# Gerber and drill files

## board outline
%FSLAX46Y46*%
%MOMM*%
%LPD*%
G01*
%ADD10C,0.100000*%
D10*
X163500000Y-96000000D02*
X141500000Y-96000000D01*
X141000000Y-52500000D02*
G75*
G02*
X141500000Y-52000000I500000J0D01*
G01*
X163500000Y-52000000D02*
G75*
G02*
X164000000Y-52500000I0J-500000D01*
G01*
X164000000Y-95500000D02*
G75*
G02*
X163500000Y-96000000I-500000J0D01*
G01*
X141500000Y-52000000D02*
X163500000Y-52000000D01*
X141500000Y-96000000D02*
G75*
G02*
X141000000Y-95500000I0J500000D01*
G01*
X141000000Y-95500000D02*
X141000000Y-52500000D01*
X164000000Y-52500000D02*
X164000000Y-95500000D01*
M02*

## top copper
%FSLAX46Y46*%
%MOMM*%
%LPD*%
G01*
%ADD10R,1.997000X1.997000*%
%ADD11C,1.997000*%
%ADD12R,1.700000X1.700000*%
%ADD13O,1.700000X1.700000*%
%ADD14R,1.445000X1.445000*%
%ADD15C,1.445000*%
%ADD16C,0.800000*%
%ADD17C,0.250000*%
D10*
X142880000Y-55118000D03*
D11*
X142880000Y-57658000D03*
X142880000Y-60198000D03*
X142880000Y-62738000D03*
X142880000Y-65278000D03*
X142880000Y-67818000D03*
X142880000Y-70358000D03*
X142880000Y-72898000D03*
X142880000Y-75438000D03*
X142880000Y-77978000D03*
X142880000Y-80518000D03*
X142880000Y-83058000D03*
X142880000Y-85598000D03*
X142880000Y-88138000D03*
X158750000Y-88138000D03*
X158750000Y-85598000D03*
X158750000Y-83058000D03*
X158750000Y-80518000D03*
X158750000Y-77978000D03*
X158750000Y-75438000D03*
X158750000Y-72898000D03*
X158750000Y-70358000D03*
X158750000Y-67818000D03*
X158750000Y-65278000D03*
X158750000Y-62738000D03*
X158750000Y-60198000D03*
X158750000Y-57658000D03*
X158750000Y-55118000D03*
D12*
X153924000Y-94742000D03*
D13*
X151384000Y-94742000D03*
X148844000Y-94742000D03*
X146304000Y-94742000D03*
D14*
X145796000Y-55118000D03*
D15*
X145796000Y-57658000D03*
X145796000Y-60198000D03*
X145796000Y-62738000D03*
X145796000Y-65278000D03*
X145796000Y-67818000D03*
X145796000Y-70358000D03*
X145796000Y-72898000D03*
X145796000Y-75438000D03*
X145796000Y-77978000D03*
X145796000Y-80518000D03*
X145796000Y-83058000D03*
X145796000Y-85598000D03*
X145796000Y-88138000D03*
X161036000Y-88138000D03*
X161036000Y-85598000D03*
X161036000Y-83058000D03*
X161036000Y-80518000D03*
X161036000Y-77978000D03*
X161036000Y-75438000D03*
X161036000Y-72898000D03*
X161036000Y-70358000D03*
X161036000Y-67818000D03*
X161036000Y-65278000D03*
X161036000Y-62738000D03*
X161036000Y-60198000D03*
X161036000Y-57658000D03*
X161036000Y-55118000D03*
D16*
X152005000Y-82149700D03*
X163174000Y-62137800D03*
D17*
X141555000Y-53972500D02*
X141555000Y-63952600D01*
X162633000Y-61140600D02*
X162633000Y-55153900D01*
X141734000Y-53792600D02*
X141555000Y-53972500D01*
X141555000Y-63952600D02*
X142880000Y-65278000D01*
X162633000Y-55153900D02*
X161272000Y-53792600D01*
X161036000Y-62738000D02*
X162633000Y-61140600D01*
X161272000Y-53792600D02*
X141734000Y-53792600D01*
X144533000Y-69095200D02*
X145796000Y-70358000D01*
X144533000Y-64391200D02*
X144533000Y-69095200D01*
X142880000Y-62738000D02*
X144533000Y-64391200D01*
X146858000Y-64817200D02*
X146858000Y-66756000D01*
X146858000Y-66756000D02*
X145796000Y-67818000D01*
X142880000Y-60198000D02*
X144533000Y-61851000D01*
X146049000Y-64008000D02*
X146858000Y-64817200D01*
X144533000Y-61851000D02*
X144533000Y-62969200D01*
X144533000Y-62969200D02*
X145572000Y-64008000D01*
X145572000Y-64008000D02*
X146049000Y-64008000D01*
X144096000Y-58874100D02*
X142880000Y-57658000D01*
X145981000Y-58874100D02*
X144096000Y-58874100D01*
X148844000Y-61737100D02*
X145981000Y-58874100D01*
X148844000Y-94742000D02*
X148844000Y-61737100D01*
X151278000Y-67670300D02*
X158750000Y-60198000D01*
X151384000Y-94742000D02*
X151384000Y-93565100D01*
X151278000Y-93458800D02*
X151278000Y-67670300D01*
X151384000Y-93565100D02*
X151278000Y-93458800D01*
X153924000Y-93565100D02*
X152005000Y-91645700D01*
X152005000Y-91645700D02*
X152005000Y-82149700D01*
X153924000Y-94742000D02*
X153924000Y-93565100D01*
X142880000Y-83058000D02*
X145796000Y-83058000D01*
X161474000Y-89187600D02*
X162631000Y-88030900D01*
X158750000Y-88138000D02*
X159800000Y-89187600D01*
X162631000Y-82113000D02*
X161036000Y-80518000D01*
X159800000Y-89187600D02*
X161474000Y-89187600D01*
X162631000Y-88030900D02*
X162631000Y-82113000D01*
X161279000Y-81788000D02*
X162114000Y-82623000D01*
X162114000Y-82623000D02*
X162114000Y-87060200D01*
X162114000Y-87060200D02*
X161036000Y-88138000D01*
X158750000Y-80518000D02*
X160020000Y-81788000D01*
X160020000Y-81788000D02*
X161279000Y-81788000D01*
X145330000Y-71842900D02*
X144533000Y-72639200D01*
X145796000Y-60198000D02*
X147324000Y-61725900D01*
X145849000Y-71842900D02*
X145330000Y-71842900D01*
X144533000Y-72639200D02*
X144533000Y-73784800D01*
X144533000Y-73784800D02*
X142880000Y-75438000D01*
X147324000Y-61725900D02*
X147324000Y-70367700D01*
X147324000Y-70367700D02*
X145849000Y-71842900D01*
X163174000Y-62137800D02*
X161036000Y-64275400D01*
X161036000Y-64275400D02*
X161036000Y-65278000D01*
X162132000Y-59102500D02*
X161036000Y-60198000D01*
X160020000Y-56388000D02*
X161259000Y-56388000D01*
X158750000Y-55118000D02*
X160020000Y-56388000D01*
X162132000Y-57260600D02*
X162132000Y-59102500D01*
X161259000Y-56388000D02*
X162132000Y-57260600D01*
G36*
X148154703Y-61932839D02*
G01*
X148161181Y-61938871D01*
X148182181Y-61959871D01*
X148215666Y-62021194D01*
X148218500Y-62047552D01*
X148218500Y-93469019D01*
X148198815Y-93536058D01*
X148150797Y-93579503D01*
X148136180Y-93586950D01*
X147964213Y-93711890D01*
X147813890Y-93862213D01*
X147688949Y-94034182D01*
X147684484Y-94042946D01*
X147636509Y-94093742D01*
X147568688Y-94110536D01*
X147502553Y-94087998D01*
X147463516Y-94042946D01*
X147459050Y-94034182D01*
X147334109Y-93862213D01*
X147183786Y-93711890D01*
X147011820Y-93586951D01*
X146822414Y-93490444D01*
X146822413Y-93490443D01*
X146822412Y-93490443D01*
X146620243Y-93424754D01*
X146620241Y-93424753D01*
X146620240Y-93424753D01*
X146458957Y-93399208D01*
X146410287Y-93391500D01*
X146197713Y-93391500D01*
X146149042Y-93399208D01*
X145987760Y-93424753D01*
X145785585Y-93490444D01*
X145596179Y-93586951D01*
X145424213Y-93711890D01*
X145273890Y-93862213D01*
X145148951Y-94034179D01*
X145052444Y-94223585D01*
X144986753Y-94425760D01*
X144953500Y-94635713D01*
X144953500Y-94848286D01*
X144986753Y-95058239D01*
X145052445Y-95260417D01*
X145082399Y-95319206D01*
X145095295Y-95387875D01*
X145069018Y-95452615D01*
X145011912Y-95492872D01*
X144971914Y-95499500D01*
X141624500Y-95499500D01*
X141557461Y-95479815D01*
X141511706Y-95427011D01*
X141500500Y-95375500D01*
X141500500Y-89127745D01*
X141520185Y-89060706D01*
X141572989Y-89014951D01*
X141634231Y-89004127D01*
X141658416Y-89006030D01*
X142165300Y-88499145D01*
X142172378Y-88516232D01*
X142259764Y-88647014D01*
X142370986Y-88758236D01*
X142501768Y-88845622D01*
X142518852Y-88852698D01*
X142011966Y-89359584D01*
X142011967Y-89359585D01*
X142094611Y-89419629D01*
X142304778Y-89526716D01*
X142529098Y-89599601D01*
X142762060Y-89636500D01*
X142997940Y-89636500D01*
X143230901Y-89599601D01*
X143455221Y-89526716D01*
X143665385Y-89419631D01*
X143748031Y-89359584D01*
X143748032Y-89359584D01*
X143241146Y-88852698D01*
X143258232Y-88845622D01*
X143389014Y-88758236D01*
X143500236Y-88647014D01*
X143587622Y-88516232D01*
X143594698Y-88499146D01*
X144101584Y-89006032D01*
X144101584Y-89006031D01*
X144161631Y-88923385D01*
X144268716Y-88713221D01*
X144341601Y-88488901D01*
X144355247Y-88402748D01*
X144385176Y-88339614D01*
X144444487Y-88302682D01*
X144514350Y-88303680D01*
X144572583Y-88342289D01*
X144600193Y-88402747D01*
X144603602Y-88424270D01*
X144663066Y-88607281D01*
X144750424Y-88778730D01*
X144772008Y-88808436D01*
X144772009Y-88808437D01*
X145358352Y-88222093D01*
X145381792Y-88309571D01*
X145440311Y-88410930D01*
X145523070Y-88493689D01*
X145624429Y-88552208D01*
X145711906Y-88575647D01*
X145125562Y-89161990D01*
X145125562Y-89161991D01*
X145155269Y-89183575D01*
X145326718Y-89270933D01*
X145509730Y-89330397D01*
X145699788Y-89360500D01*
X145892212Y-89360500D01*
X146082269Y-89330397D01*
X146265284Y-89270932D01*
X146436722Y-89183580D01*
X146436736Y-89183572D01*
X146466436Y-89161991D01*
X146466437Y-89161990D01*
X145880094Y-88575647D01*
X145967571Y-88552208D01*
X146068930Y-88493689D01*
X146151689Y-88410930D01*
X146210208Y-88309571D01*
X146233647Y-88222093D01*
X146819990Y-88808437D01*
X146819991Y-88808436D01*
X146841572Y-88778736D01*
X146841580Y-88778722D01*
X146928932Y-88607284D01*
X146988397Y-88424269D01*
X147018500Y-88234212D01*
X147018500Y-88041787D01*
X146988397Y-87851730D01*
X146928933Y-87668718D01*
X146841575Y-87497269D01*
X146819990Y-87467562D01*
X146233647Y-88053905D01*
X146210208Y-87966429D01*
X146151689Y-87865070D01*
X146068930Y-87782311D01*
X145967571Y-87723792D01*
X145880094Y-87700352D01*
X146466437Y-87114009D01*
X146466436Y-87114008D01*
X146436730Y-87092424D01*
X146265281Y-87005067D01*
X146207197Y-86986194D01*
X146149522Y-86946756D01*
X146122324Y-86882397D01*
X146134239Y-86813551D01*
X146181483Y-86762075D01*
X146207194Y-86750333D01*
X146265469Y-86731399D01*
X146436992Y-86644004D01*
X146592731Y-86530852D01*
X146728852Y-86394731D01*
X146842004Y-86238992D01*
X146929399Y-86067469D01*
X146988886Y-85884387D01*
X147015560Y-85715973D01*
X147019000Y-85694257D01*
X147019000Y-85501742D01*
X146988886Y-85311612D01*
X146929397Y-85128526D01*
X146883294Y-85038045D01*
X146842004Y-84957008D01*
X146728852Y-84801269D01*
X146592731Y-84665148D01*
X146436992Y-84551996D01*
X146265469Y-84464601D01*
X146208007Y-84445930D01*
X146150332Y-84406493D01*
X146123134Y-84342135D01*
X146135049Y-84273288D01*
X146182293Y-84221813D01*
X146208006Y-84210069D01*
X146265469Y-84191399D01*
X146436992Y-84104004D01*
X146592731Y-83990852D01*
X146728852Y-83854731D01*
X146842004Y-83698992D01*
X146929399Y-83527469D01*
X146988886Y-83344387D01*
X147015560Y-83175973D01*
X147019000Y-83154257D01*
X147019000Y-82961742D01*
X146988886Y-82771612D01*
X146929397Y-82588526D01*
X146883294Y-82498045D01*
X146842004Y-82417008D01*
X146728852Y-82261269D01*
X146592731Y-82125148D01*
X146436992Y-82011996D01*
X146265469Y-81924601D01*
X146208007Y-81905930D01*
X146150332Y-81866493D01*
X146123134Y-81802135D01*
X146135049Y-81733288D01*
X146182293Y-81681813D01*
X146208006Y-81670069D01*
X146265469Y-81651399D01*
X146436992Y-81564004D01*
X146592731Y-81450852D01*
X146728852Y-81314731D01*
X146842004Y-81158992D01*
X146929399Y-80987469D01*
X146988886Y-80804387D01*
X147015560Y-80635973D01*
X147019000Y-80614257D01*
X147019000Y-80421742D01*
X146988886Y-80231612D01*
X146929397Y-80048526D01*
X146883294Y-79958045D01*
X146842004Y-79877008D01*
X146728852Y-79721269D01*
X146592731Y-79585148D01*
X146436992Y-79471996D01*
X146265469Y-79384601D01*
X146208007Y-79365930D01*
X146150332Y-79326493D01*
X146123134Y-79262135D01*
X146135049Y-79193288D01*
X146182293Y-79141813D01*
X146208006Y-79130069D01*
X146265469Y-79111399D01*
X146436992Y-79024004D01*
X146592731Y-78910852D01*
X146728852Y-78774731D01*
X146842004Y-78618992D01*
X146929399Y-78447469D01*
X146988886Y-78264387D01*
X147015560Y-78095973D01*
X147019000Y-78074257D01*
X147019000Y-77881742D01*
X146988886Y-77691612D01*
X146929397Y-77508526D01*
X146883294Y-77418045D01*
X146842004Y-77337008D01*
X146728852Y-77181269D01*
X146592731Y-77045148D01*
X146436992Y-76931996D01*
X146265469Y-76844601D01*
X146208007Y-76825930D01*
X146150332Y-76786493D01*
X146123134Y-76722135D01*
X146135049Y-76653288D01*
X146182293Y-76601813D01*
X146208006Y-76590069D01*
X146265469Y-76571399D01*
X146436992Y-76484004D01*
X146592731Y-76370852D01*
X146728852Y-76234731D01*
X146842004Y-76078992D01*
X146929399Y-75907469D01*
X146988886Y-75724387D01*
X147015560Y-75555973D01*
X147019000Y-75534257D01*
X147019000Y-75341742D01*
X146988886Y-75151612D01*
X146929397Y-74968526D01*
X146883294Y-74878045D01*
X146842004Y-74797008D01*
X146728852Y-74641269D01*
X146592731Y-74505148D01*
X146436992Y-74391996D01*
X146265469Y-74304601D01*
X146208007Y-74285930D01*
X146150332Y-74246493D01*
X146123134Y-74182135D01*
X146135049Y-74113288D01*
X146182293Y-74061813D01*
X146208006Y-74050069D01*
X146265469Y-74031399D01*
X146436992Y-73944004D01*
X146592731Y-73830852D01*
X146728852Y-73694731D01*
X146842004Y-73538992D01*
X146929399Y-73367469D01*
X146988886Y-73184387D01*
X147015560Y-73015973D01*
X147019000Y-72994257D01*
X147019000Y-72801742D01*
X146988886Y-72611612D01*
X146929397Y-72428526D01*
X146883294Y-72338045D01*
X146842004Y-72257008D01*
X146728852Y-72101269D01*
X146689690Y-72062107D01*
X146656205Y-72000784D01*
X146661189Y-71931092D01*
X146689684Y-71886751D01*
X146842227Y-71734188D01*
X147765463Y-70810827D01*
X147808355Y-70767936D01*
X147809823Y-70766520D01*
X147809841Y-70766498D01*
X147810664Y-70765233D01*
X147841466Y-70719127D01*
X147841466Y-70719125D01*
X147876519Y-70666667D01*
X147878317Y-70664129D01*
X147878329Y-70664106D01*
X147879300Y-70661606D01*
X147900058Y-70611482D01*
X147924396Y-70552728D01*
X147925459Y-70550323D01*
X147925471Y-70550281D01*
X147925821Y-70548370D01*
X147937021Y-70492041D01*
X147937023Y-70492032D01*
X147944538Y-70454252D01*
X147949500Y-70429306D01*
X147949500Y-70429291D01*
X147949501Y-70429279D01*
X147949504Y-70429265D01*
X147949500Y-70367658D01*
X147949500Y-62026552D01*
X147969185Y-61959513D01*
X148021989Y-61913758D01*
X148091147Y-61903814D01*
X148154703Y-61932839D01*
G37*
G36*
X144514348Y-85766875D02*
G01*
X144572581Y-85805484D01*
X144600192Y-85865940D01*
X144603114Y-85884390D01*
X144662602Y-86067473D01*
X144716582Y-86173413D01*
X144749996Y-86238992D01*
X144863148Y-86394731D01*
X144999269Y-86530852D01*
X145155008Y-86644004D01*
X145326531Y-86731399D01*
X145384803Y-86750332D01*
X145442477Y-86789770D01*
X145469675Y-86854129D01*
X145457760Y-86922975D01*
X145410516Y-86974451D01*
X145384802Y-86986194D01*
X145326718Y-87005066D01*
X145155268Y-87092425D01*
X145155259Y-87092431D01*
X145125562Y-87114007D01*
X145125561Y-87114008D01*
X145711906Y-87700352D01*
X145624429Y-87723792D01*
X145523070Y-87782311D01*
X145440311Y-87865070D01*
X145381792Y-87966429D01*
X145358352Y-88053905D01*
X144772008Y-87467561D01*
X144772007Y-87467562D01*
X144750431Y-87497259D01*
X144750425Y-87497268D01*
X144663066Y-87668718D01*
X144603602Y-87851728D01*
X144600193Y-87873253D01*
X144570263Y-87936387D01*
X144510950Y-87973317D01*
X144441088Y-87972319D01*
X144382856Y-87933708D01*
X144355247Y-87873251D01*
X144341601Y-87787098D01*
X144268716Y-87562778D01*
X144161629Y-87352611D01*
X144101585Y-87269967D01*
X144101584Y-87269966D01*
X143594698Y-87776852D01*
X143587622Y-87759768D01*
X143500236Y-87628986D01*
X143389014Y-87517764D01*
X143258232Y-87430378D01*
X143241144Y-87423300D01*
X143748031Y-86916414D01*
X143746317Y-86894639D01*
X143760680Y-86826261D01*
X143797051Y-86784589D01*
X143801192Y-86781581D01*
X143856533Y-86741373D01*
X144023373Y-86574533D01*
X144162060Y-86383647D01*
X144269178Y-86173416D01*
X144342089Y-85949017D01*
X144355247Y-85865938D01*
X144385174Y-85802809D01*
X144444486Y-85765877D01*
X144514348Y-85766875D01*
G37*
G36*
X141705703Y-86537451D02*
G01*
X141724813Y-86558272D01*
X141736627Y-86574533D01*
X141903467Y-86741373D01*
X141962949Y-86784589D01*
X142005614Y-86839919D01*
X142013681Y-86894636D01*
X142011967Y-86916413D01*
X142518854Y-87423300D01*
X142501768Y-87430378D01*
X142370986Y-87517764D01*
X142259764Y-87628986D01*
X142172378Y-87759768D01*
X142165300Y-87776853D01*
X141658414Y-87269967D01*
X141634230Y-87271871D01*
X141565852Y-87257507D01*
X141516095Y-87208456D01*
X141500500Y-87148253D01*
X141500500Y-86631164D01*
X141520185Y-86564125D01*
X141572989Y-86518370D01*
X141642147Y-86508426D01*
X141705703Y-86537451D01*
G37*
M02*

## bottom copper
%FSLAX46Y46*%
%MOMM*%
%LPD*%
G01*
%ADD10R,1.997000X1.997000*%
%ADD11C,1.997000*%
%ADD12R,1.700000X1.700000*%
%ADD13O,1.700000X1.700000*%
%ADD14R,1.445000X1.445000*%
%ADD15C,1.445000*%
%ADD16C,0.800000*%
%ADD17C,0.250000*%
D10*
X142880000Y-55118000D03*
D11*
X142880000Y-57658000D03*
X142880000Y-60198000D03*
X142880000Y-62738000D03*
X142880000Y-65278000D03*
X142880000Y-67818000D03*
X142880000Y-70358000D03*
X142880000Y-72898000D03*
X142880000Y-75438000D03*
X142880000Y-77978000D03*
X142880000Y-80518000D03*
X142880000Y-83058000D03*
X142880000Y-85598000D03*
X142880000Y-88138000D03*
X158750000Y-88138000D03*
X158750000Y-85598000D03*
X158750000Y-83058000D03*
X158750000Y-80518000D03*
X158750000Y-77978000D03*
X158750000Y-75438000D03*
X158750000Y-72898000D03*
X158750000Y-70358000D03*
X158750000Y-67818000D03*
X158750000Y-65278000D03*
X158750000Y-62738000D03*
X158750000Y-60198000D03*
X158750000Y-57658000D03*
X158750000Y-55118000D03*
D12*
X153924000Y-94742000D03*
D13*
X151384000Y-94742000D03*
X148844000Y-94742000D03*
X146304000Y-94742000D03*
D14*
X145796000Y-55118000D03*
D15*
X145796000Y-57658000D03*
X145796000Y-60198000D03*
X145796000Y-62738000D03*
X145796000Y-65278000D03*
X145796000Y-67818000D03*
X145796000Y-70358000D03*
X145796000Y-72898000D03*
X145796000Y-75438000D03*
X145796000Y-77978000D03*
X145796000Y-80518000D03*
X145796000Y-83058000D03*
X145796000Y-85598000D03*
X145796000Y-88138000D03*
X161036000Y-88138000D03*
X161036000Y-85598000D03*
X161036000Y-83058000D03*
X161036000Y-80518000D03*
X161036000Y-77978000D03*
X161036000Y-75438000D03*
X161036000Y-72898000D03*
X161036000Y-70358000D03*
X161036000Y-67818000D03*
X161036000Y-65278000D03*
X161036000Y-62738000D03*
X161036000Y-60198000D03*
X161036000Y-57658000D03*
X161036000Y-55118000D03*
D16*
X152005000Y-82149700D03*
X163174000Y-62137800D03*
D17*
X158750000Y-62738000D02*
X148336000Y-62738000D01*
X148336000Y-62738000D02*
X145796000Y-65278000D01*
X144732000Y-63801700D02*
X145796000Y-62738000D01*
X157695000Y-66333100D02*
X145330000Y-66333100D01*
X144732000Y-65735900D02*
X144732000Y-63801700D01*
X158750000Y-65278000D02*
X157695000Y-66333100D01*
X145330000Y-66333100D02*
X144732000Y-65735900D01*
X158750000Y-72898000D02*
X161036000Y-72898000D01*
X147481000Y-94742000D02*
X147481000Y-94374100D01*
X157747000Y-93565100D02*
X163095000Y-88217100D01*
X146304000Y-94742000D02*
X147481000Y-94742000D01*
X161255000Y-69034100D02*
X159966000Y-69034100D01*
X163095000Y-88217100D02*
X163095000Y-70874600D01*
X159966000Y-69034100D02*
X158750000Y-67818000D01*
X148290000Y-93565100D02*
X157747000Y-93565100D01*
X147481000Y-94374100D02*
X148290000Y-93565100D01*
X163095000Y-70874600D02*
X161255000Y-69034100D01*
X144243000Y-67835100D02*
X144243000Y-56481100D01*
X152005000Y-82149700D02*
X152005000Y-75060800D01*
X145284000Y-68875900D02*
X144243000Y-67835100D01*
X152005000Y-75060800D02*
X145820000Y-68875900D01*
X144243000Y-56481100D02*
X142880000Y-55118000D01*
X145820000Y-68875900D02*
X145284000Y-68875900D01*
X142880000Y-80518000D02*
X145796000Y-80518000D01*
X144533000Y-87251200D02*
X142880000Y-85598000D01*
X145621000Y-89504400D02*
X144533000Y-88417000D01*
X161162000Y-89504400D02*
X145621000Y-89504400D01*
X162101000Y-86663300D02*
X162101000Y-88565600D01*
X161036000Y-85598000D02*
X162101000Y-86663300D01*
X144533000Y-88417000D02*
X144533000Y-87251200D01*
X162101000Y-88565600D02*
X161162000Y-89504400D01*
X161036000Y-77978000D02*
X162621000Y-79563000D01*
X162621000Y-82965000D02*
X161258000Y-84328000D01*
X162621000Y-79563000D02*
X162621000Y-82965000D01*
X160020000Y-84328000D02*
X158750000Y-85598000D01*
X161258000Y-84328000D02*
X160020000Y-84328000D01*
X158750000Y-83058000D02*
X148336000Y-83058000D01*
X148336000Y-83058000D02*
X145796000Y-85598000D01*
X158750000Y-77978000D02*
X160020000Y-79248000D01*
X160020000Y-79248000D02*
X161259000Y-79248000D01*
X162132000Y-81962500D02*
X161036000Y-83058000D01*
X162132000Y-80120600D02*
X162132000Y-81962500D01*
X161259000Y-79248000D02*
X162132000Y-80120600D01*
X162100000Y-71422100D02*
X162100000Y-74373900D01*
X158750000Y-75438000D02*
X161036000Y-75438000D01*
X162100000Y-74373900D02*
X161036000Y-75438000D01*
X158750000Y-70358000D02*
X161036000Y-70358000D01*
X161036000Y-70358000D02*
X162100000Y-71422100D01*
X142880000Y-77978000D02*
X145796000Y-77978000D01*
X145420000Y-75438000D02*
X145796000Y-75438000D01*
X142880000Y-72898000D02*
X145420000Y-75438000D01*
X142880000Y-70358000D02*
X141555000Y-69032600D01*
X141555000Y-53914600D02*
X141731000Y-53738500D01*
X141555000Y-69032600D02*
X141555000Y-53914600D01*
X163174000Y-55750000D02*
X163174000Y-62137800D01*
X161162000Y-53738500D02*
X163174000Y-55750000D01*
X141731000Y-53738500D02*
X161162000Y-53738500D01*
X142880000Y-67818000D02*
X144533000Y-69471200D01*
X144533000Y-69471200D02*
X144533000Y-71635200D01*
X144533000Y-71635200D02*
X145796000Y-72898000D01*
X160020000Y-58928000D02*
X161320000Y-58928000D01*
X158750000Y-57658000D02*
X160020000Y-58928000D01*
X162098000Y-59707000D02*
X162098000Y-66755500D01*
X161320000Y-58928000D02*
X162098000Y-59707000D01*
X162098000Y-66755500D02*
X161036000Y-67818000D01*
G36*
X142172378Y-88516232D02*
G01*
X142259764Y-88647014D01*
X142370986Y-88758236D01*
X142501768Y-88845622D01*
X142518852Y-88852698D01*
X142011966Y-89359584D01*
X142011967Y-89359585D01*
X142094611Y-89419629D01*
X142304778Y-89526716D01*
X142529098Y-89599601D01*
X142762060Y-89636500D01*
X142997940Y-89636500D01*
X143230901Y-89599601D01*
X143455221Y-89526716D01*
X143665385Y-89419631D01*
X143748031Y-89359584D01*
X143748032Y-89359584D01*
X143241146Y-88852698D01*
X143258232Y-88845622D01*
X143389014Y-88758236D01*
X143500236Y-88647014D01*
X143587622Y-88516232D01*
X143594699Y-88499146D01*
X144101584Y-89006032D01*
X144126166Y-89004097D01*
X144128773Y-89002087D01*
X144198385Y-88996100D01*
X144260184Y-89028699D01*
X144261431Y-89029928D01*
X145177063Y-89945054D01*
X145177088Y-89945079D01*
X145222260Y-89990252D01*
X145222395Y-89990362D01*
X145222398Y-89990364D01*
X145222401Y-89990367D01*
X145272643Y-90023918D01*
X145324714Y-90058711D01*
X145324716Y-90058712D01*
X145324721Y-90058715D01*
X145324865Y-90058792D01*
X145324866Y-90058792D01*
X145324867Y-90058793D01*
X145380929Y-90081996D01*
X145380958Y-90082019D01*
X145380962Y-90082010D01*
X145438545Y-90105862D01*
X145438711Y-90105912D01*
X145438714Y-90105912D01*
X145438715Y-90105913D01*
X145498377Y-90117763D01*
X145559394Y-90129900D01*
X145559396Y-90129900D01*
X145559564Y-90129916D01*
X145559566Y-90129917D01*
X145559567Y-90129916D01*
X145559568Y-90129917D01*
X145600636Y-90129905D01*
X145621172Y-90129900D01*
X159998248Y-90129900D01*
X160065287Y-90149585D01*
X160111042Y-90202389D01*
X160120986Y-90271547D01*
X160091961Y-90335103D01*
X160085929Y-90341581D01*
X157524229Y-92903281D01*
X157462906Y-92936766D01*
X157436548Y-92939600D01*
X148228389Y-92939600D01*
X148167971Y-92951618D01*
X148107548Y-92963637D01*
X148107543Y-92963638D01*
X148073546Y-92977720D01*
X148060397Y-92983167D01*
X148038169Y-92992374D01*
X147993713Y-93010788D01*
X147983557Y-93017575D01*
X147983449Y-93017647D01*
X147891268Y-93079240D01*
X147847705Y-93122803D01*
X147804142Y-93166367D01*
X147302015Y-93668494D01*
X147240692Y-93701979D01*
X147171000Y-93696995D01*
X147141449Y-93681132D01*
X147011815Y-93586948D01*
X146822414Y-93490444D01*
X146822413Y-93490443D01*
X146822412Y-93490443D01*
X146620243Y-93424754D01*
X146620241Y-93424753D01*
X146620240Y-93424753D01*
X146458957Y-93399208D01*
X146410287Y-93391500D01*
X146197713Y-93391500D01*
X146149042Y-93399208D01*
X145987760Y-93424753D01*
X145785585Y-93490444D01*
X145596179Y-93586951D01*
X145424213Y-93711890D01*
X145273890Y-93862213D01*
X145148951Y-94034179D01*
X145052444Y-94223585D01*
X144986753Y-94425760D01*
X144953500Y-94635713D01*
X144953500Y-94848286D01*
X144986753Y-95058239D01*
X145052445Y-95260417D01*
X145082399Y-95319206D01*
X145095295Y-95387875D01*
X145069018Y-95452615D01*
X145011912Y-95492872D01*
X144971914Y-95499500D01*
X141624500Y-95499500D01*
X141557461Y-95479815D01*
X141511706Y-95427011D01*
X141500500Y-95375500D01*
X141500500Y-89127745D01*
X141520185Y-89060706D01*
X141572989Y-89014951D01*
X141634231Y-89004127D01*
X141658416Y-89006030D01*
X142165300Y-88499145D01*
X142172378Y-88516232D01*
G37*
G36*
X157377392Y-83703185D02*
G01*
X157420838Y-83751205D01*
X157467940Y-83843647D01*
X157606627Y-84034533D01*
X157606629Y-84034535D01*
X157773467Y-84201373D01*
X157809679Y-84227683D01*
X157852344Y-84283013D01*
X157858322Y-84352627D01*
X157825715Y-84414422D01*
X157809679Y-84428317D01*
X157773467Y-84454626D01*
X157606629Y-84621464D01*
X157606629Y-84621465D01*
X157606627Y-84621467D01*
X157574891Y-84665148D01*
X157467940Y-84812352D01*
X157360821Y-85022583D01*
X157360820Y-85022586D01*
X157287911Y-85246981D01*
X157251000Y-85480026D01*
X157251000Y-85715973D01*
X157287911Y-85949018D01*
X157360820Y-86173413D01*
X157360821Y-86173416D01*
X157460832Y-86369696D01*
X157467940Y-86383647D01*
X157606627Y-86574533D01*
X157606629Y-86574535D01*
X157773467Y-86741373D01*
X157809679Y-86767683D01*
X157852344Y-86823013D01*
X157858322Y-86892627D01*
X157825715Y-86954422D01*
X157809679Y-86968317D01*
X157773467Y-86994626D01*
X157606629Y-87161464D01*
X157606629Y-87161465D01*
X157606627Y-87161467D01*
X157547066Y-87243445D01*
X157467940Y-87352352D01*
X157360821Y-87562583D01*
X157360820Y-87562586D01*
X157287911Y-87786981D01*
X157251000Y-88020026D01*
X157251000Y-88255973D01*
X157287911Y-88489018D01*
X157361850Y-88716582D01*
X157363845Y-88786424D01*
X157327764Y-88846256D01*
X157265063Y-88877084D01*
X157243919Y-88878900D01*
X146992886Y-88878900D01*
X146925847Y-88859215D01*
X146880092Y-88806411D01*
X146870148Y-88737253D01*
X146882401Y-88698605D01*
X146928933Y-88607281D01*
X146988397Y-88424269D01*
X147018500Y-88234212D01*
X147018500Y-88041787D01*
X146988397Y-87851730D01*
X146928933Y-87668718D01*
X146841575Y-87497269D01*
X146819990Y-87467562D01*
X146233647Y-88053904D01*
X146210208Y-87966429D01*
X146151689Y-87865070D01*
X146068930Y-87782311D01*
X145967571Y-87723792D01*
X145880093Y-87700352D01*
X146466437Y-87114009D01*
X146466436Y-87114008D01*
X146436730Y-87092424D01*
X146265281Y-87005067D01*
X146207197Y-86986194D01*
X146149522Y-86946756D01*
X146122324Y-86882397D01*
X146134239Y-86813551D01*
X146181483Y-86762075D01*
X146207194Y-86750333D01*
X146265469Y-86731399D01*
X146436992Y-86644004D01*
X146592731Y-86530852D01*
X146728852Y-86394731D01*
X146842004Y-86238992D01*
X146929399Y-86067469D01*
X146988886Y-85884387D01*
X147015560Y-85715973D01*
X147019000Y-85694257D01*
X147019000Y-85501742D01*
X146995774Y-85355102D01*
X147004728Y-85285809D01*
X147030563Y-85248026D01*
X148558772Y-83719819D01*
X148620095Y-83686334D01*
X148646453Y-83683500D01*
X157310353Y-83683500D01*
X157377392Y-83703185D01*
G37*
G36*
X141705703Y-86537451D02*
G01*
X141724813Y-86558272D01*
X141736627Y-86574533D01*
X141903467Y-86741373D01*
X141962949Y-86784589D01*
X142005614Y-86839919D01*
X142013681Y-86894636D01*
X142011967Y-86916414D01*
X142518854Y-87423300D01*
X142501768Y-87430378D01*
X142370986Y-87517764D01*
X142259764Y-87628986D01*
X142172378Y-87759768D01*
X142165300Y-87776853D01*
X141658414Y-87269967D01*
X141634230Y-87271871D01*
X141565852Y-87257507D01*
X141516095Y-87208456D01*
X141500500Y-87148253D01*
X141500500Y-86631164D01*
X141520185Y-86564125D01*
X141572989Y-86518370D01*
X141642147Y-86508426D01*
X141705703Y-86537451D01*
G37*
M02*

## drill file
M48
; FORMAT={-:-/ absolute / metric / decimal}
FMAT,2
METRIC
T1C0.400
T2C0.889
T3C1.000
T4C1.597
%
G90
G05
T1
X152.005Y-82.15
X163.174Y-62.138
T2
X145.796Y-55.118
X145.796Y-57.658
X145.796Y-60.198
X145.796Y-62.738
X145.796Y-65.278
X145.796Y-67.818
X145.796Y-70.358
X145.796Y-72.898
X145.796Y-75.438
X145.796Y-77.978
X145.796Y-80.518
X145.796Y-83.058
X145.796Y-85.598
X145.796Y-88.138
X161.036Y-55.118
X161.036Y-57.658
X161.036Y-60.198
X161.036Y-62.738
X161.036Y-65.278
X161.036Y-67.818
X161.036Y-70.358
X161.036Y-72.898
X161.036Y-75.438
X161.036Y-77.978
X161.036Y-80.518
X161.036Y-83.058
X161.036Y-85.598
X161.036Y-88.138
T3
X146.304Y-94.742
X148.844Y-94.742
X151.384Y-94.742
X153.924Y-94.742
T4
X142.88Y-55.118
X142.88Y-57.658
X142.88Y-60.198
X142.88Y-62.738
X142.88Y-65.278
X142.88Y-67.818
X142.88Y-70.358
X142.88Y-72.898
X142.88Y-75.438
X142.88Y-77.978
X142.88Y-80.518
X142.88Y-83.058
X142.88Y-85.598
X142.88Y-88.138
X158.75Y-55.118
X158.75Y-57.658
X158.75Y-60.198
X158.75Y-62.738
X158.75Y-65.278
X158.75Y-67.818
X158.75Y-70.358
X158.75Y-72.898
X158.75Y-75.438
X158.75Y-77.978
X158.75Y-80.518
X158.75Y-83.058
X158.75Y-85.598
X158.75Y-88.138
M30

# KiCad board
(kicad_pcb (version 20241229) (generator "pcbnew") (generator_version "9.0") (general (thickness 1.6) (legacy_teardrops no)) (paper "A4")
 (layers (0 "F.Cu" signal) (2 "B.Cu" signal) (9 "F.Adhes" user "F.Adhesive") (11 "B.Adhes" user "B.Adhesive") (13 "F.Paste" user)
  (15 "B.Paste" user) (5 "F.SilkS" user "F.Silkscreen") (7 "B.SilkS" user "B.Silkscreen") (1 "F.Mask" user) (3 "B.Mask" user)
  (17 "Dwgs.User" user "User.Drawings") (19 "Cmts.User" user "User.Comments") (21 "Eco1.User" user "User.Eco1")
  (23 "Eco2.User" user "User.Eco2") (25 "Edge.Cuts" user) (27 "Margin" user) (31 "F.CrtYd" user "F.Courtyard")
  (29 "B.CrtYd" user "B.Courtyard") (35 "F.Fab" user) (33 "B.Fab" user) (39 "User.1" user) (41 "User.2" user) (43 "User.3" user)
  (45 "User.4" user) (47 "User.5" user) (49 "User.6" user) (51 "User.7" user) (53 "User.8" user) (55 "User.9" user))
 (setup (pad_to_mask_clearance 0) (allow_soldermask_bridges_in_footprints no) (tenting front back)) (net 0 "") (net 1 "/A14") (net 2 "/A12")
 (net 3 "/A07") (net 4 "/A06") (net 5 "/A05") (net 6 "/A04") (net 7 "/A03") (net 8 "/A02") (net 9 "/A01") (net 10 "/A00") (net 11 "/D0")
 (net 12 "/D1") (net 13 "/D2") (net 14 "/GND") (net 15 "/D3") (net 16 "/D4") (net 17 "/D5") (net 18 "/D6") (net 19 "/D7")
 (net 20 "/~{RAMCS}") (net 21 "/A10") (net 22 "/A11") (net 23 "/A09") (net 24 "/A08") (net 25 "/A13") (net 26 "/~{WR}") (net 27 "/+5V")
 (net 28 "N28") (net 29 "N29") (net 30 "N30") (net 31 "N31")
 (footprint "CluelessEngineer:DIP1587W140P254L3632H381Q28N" (layer "F.Cu") (at 150.815 71.628)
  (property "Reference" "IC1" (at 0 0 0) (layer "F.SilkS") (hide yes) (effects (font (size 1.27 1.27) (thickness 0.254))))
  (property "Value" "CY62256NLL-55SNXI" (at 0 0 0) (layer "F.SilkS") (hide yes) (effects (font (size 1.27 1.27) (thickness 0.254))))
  (pad "1" thru_hole rect (at -7.935 -16.51) (size 1.997 1.997) (drill 1.597) (layers "*.Cu" "*.Mask") (remove_unused_layers no)
   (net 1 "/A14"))
  (pad "2" thru_hole circle (at -7.935 -13.97) (size 1.997 1.997) (drill 1.597) (layers "*.Cu" "*.Mask") (remove_unused_layers no)
   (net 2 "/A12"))
  (pad "3" thru_hole circle (at -7.935 -11.43) (size 1.997 1.997) (drill 1.597) (layers "*.Cu" "*.Mask") (remove_unused_layers no)
   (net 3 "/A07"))
  (pad "4" thru_hole circle (at -7.935 -8.89) (size 1.997 1.997) (drill 1.597) (layers "*.Cu" "*.Mask") (remove_unused_layers no)
   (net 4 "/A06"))
  (pad "5" thru_hole circle (at -7.935 -6.35) (size 1.997 1.997) (drill 1.597) (layers "*.Cu" "*.Mask") (remove_unused_layers no)
   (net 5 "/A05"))
  (pad "6" thru_hole circle (at -7.935 -3.81) (size 1.997 1.997) (drill 1.597) (layers "*.Cu" "*.Mask") (remove_unused_layers no)
   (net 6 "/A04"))
  (pad "7" thru_hole circle (at -7.935 -1.27) (size 1.997 1.997) (drill 1.597) (layers "*.Cu" "*.Mask") (remove_unused_layers no)
   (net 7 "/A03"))
  (pad "8" thru_hole circle (at -7.935 1.27) (size 1.997 1.997) (drill 1.597) (layers "*.Cu" "*.Mask") (remove_unused_layers no)
   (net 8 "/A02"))
  (pad "9" thru_hole circle (at -7.935 3.81) (size 1.997 1.997) (drill 1.597) (layers "*.Cu" "*.Mask") (remove_unused_layers no)
   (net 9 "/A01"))
  (pad "10" thru_hole circle (at -7.935 6.35) (size 1.997 1.997) (drill 1.597) (layers "*.Cu" "*.Mask") (remove_unused_layers no)
   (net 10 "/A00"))
  (pad "11" thru_hole circle (at -7.935 8.89) (size 1.997 1.997) (drill 1.597) (layers "*.Cu" "*.Mask") (remove_unused_layers no)
   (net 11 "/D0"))
  (pad "12" thru_hole circle (at -7.935 11.43) (size 1.997 1.997) (drill 1.597) (layers "*.Cu" "*.Mask") (remove_unused_layers no)
   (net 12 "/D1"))
  (pad "13" thru_hole circle (at -7.935 13.97) (size 1.997 1.997) (drill 1.597) (layers "*.Cu" "*.Mask") (remove_unused_layers no)
   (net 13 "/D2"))
  (pad "14" thru_hole circle (at -7.935 16.51) (size 1.997 1.997) (drill 1.597) (layers "*.Cu" "*.Mask") (remove_unused_layers no)
   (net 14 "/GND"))
  (pad "15" thru_hole circle (at 7.935 16.51) (size 1.997 1.997) (drill 1.597) (layers "*.Cu" "*.Mask") (remove_unused_layers no)
   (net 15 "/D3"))
  (pad "16" thru_hole circle (at 7.935 13.97) (size 1.997 1.997) (drill 1.597) (layers "*.Cu" "*.Mask") (remove_unused_layers no)
   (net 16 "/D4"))
  (pad "17" thru_hole circle (at 7.935 11.43) (size 1.997 1.997) (drill 1.597) (layers "*.Cu" "*.Mask") (remove_unused_layers no)
   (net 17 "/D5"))
  (pad "18" thru_hole circle (at 7.935 8.89) (size 1.997 1.997) (drill 1.597) (layers "*.Cu" "*.Mask") (remove_unused_layers no)
   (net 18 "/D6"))
  (pad "19" thru_hole circle (at 7.935 6.35) (size 1.997 1.997) (drill 1.597) (layers "*.Cu" "*.Mask") (remove_unused_layers no)
   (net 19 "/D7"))
  (pad "20" thru_hole circle (at 7.935 3.81) (size 1.997 1.997) (drill 1.597) (layers "*.Cu" "*.Mask") (remove_unused_layers no)
   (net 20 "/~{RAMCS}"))
  (pad "21" thru_hole circle (at 7.935 1.27) (size 1.997 1.997) (drill 1.597) (layers "*.Cu" "*.Mask") (remove_unused_layers no)
   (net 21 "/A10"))
  (pad "22" thru_hole circle (at 7.935 -1.27) (size 1.997 1.997) (drill 1.597) (layers "*.Cu" "*.Mask") (remove_unused_layers no)
   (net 20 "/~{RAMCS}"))
  (pad "23" thru_hole circle (at 7.935 -3.81) (size 1.997 1.997) (drill 1.597) (layers "*.Cu" "*.Mask") (remove_unused_layers no)
   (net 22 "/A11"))
  (pad "24" thru_hole circle (at 7.935 -6.35) (size 1.997 1.997) (drill 1.597) (layers "*.Cu" "*.Mask") (remove_unused_layers no)
   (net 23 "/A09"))
  (pad "25" thru_hole circle (at 7.935 -8.89) (size 1.997 1.997) (drill 1.597) (layers "*.Cu" "*.Mask") (remove_unused_layers no)
   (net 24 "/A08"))
  (pad "26" thru_hole circle (at 7.935 -11.43) (size 1.997 1.997) (drill 1.597) (layers "*.Cu" "*.Mask") (remove_unused_layers no)
   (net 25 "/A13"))
  (pad "27" thru_hole circle (at 7.935 -13.97) (size 1.997 1.997) (drill 1.597) (layers "*.Cu" "*.Mask") (remove_unused_layers no)
   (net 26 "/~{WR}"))
  (pad "28" thru_hole circle (at 7.935 -16.51) (size 1.997 1.997) (drill 1.597) (layers "*.Cu" "*.Mask") (remove_unused_layers no)
   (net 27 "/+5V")))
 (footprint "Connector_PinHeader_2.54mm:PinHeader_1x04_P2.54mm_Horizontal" (layer "F.Cu") (at 153.924 94.742 -90)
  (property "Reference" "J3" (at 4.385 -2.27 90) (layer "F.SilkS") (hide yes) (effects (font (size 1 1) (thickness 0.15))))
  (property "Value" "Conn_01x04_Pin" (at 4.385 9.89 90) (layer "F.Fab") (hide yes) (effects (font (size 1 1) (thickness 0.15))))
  (pad "1" thru_hole rect (at 0 0 270) (size 1.7 1.7) (drill 1) (layers "*.Cu" "*.Mask") (remove_unused_layers no) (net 1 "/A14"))
  (pad "2" thru_hole oval (at 0 2.54 270) (size 1.7 1.7) (drill 1) (layers "*.Cu" "*.Mask") (remove_unused_layers no) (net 25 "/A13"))
  (pad "3" thru_hole oval (at 0 5.08 270) (size 1.7 1.7) (drill 1) (layers "*.Cu" "*.Mask") (remove_unused_layers no) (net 2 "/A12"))
  (pad "4" thru_hole oval (at 0 7.62 270) (size 1.7 1.7) (drill 1) (layers "*.Cu" "*.Mask") (remove_unused_layers no) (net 22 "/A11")))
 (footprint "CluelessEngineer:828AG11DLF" (layer "F.Cu") (at 145.796 55.118 -90)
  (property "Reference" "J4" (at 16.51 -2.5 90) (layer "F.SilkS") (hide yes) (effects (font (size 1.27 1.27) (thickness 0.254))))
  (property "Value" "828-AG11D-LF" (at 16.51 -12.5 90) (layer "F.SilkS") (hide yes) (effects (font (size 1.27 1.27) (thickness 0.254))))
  (pad "1" thru_hole rect (at 0 0 270) (size 1.445 1.445) (drill 0.889) (layers "*.Cu" "*.Mask") (remove_unused_layers no) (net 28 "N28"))
  (pad "2" thru_hole circle (at 2.54 0 270) (size 1.445 1.445) (drill 0.889) (layers "*.Cu" "*.Mask") (remove_unused_layers no)
   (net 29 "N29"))
  (pad "3" thru_hole circle (at 5.08 0 270) (size 1.445 1.445) (drill 0.889) (layers "*.Cu" "*.Mask") (remove_unused_layers no)
   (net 9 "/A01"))
  (pad "4" thru_hole circle (at 7.62 0 270) (size 1.445 1.445) (drill 0.889) (layers "*.Cu" "*.Mask") (remove_unused_layers no)
   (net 23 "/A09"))
  (pad "5" thru_hole circle (at 10.16 0 270) (size 1.445 1.445) (drill 0.889) (layers "*.Cu" "*.Mask") (remove_unused_layers no)
   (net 24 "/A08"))
  (pad "6" thru_hole circle (at 12.7 0 270) (size 1.445 1.445) (drill 0.889) (layers "*.Cu" "*.Mask") (remove_unused_layers no)
   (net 3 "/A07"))
  (pad "7" thru_hole circle (at 15.24 0 270) (size 1.445 1.445) (drill 0.889) (layers "*.Cu" "*.Mask") (remove_unused_layers no)
   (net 4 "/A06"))
  (pad "8" thru_hole circle (at 17.78 0 270) (size 1.445 1.445) (drill 0.889) (layers "*.Cu" "*.Mask") (remove_unused_layers no)
   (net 6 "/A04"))
  (pad "9" thru_hole circle (at 20.32 0 270) (size 1.445 1.445) (drill 0.889) (layers "*.Cu" "*.Mask") (remove_unused_layers no)
   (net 8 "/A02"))
  (pad "10" thru_hole circle (at 22.86 0 270) (size 1.445 1.445) (drill 0.889) (layers "*.Cu" "*.Mask") (remove_unused_layers no)
   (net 10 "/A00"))
  (pad "11" thru_hole circle (at 25.4 0 270) (size 1.445 1.445) (drill 0.889) (layers "*.Cu" "*.Mask") (remove_unused_layers no)
   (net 11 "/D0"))
  (pad "12" thru_hole circle (at 27.94 0 270) (size 1.445 1.445) (drill 0.889) (layers "*.Cu" "*.Mask") (remove_unused_layers no)
   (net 12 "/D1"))
  (pad "13" thru_hole circle (at 30.48 0 270) (size 1.445 1.445) (drill 0.889) (layers "*.Cu" "*.Mask") (remove_unused_layers no)
   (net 17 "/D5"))
  (pad "14" thru_hole circle (at 33.02 0 270) (size 1.445 1.445) (drill 0.889) (layers "*.Cu" "*.Mask") (remove_unused_layers no)
   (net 14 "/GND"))
  (pad "15" thru_hole circle (at 33.02 -15.24 270) (size 1.445 1.445) (drill 0.889) (layers "*.Cu" "*.Mask") (remove_unused_layers no)
   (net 18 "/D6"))
  (pad "16" thru_hole circle (at 30.48 -15.24 270) (size 1.445 1.445) (drill 0.889) (layers "*.Cu" "*.Mask") (remove_unused_layers no)
   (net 13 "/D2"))
  (pad "17" thru_hole circle (at 27.94 -15.24 270) (size 1.445 1.445) (drill 0.889) (layers "*.Cu" "*.Mask") (remove_unused_layers no)
   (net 19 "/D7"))
  (pad "18" thru_hole circle (at 25.4 -15.24 270) (size 1.445 1.445) (drill 0.889) (layers "*.Cu" "*.Mask") (remove_unused_layers no)
   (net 15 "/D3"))
  (pad "19" thru_hole circle (at 22.86 -15.24 270) (size 1.445 1.445) (drill 0.889) (layers "*.Cu" "*.Mask") (remove_unused_layers no)
   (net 16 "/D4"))
  (pad "20" thru_hole circle (at 20.32 -15.24 270) (size 1.445 1.445) (drill 0.889) (layers "*.Cu" "*.Mask") (remove_unused_layers no)
   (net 20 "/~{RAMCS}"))
  (pad "21" thru_hole circle (at 17.78 -15.24 270) (size 1.445 1.445) (drill 0.889) (layers "*.Cu" "*.Mask") (remove_unused_layers no)
   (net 21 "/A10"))
  (pad "22" thru_hole circle (at 15.24 -15.24 270) (size 1.445 1.445) (drill 0.889) (layers "*.Cu" "*.Mask") (remove_unused_layers no)
   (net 20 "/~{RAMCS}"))
  (pad "23" thru_hole circle (at 12.7 -15.24 270) (size 1.445 1.445) (drill 0.889) (layers "*.Cu" "*.Mask") (remove_unused_layers no)
   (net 26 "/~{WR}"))
  (pad "24" thru_hole circle (at 10.16 -15.24 270) (size 1.445 1.445) (drill 0.889) (layers "*.Cu" "*.Mask") (remove_unused_layers no)
   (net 7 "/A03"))
  (pad "25" thru_hole circle (at 7.62 -15.24 270) (size 1.445 1.445) (drill 0.889) (layers "*.Cu" "*.Mask") (remove_unused_layers no)
   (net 5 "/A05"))
  (pad "26" thru_hole circle (at 5.08 -15.24 270) (size 1.445 1.445) (drill 0.889) (layers "*.Cu" "*.Mask") (remove_unused_layers no)
   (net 27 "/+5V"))
  (pad "27" thru_hole circle (at 2.54 -15.24 270) (size 1.445 1.445) (drill 0.889) (layers "*.Cu" "*.Mask") (remove_unused_layers no)
   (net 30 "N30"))
  (pad "28" thru_hole circle (at 0 -15.24 270) (size 1.445 1.445) (drill 0.889) (layers "*.Cu" "*.Mask") (remove_unused_layers no)
   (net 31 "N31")))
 (gr_line (start 163.5 96) (end 141.5 96) (stroke (width 0.1) (type default)) (layer "Edge.Cuts"))
 (gr_arc (start 141 52.5) (mid 141.146447 52.146447) (end 141.5 52) (stroke (width 0.1) (type default)) (layer "Edge.Cuts"))
 (gr_arc (start 163.5 52) (mid 163.853553 52.146447) (end 164 52.5) (stroke (width 0.1) (type default)) (layer "Edge.Cuts"))
 (gr_arc (start 164 95.5) (mid 163.853553 95.853553) (end 163.5 96) (stroke (width 0.1) (type default)) (layer "Edge.Cuts"))
 (gr_line (start 141.5 52) (end 163.5 52) (stroke (width 0.1) (type default)) (layer "Edge.Cuts"))
 (gr_arc (start 141.5 96) (mid 141.146447 95.853553) (end 141 95.5) (stroke (width 0.1) (type default)) (layer "Edge.Cuts"))
 (gr_line (start 141 95.5) (end 141 52.5) (stroke (width 0.1) (type default)) (layer "Edge.Cuts"))
 (gr_line (start 164 52.5) (end 164 95.5) (stroke (width 0.1) (type default)) (layer "Edge.Cuts"))
 (segment (start 141.555 53.9725) (end 141.555 63.9526) (width 0.25) (layer "F.Cu") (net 5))
 (segment (start 162.633 61.1406) (end 162.633 55.1539) (width 0.25) (layer "F.Cu") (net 5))
 (segment (start 141.734 53.7926) (end 141.555 53.9725) (width 0.25) (layer "F.Cu") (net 5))
 (segment (start 141.555 63.9526) (end 142.88 65.278) (width 0.25) (layer "F.Cu") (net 5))
 (segment (start 162.633 55.1539) (end 161.272 53.7926) (width 0.25) (layer "F.Cu") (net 5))
 (segment (start 161.036 62.738) (end 162.633 61.1406) (width 0.25) (layer "F.Cu") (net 5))
 (segment (start 161.272 53.7926) (end 141.734 53.7926) (width 0.25) (layer "F.Cu") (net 5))
 (segment (start 144.533 69.0952) (end 145.796 70.358) (width 0.25) (layer "F.Cu") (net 4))
 (segment (start 144.533 64.3912) (end 144.533 69.0952) (width 0.25) (layer "F.Cu") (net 4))
 (segment (start 142.88 62.738) (end 144.533 64.3912) (width 0.25) (layer "F.Cu") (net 4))
 (segment (start 146.858 64.8172) (end 146.858 66.756) (width 0.25) (layer "F.Cu") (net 3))
 (segment (start 146.858 66.756) (end 145.796 67.818) (width 0.25) (layer "F.Cu") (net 3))
 (segment (start 142.88 60.198) (end 144.533 61.851) (width 0.25) (layer "F.Cu") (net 3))
 (segment (start 146.049 64.008) (end 146.858 64.8172) (width 0.25) (layer "F.Cu") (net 3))
 (segment (start 144.533 61.851) (end 144.533 62.9692) (width 0.25) (layer "F.Cu") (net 3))
 (segment (start 144.533 62.9692) (end 145.572 64.008) (width 0.25) (layer "F.Cu") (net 3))
 (segment (start 145.572 64.008) (end 146.049 64.008) (width 0.25) (layer "F.Cu") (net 3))
 (segment (start 158.75 62.738) (end 148.336 62.738) (width 0.25) (layer "B.Cu") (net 24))
 (segment (start 148.336 62.738) (end 145.796 65.278) (width 0.25) (layer "B.Cu") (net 24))
 (segment (start 144.732 63.8017) (end 145.796 62.738) (width 0.25) (layer "B.Cu") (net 23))
 (segment (start 157.695 66.3331) (end 145.33 66.3331) (width 0.25) (layer "B.Cu") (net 23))
 (segment (start 144.732 65.7359) (end 144.732 63.8017) (width 0.25) (layer "B.Cu") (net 23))
 (segment (start 158.75 65.278) (end 157.695 66.3331) (width 0.25) (layer "B.Cu") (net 23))
 (segment (start 145.33 66.3331) (end 144.732 65.7359) (width 0.25) (layer "B.Cu") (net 23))
 (segment (start 158.75 72.898) (end 161.036 72.898) (width 0.25) (layer "B.Cu") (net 21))
 (segment (start 147.481 94.742) (end 147.481 94.3741) (width 0.25) (layer "B.Cu") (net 22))
 (segment (start 157.747 93.5651) (end 163.095 88.2171) (width 0.25) (layer "B.Cu") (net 22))
 (segment (start 146.304 94.742) (end 147.481 94.742) (width 0.25) (layer "B.Cu") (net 22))
 (segment (start 161.255 69.0341) (end 159.966 69.0341) (width 0.25) (layer "B.Cu") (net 22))
 (segment (start 163.095 88.2171) (end 163.095 70.8746) (width 0.25) (layer "B.Cu") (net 22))
 (segment (start 159.966 69.0341) (end 158.75 67.818) (width 0.25) (layer "B.Cu") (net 22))
 (segment (start 148.29 93.5651) (end 157.747 93.5651) (width 0.25) (layer "B.Cu") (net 22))
 (segment (start 147.481 94.3741) (end 148.29 93.5651) (width 0.25) (layer "B.Cu") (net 22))
 (segment (start 163.095 70.8746) (end 161.255 69.0341) (width 0.25) (layer "B.Cu") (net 22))
 (segment (start 144.096 58.8741) (end 142.88 57.658) (width 0.25) (layer "F.Cu") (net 2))
 (segment (start 145.981 58.8741) (end 144.096 58.8741) (width 0.25) (layer "F.Cu") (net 2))
 (segment (start 148.844 61.7371) (end 145.981 58.8741) (width 0.25) (layer "F.Cu") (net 2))
 (segment (start 148.844 94.742) (end 148.844 61.7371) (width 0.25) (layer "F.Cu") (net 2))
 (segment (start 151.278 67.6703) (end 158.75 60.198) (width 0.25) (layer "F.Cu") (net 25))
 (segment (start 151.384 94.742) (end 151.384 93.5651) (width 0.25) (layer "F.Cu") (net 25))
 (segment (start 151.278 93.4588) (end 151.278 67.6703) (width 0.25) (layer "F.Cu") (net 25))
 (segment (start 151.384 93.5651) (end 151.278 93.4588) (width 0.25) (layer "F.Cu") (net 25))
 (segment (start 153.924 93.5651) (end 152.005 91.6457) (width 0.25) (layer "F.Cu") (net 1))
 (segment (start 152.005 91.6457) (end 152.005 82.1497) (width 0.25) (layer "F.Cu") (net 1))
 (segment (start 153.924 94.742) (end 153.924 93.5651) (width 0.25) (layer "F.Cu") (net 1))
 (via (at 152.005 82.1497) (size 0.8) (drill 0.4) (layers "F.Cu" "B.Cu") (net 1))
 (segment (start 144.243 67.8351) (end 144.243 56.4811) (width 0.25) (layer "B.Cu") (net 1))
 (segment (start 152.005 82.1497) (end 152.005 75.0608) (width 0.25) (layer "B.Cu") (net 1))
 (segment (start 145.284 68.8759) (end 144.243 67.8351) (width 0.25) (layer "B.Cu") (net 1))
 (segment (start 152.005 75.0608) (end 145.82 68.8759) (width 0.25) (layer "B.Cu") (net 1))
 (segment (start 144.243 56.4811) (end 142.88 55.118) (width 0.25) (layer "B.Cu") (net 1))
 (segment (start 145.82 68.8759) (end 145.284 68.8759) (width 0.25) (layer "B.Cu") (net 1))
 (segment (start 142.88 80.518) (end 145.796 80.518) (width 0.25) (layer "B.Cu") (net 11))
 (segment (start 142.88 83.058) (end 145.796 83.058) (width 0.25) (layer "F.Cu") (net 12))
 (segment (start 144.533 87.2512) (end 142.88 85.598) (width 0.25) (layer "B.Cu") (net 13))
 (segment (start 145.621 89.5044) (end 144.533 88.417) (width 0.25) (layer "B.Cu") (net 13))
 (segment (start 161.162 89.5044) (end 145.621 89.5044) (width 0.25) (layer "B.Cu") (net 13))
 (segment (start 162.101 86.6633) (end 162.101 88.5656) (width 0.25) (layer "B.Cu") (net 13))
 (segment (start 161.036 85.598) (end 162.101 86.6633) (width 0.25) (layer "B.Cu") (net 13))
 (segment (start 144.533 88.417) (end 144.533 87.2512) (width 0.25) (layer "B.Cu") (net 13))
 (segment (start 162.101 88.5656) (end 161.162 89.5044) (width 0.25) (layer "B.Cu") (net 13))
 (segment (start 161.474 89.1876) (end 162.631 88.0309) (width 0.25) (layer "F.Cu") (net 15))
 (segment (start 158.75 88.138) (end 159.8 89.1876) (width 0.25) (layer "F.Cu") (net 15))
 (segment (start 162.631 82.113) (end 161.036 80.518) (width 0.25) (layer "F.Cu") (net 15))
 (segment (start 159.8 89.1876) (end 161.474 89.1876) (width 0.25) (layer "F.Cu") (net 15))
 (segment (start 162.631 88.0309) (end 162.631 82.113) (width 0.25) (layer "F.Cu") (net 15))
 (segment (start 161.036 77.978) (end 162.621 79.563) (width 0.25) (layer "B.Cu") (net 16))
 (segment (start 162.621 82.965) (end 161.258 84.328) (width 0.25) (layer "B.Cu") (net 16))
 (segment (start 162.621 79.563) (end 162.621 82.965) (width 0.25) (layer "B.Cu") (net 16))
 (segment (start 160.02 84.328) (end 158.75 85.598) (width 0.25) (layer "B.Cu") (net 16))
 (segment (start 161.258 84.328) (end 160.02 84.328) (width 0.25) (layer "B.Cu") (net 16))
 (segment (start 158.75 83.058) (end 148.336 83.058) (width 0.25) (layer "B.Cu") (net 17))
 (segment (start 148.336 83.058) (end 145.796 85.598) (width 0.25) (layer "B.Cu") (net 17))
 (segment (start 161.279 81.788) (end 162.114 82.623) (width 0.25) (layer "F.Cu") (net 18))
 (segment (start 162.114 82.623) (end 162.114 87.0602) (width 0.25) (layer "F.Cu") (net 18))
 (segment (start 162.114 87.0602) (end 161.036 88.138) (width 0.25) (layer "F.Cu") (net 18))
 (segment (start 158.75 80.518) (end 160.02 81.788) (width 0.25) (layer "F.Cu") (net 18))
 (segment (start 160.02 81.788) (end 161.279 81.788) (width 0.25) (layer "F.Cu") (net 18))
 (segment (start 158.75 77.978) (end 160.02 79.248) (width 0.25) (layer "B.Cu") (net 19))
 (segment (start 160.02 79.248) (end 161.259 79.248) (width 0.25) (layer "B.Cu") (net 19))
 (segment (start 162.132 81.9625) (end 161.036 83.058) (width 0.25) (layer "B.Cu") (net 19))
 (segment (start 162.132 80.1206) (end 162.132 81.9625) (width 0.25) (layer "B.Cu") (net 19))
 (segment (start 161.259 79.248) (end 162.132 80.1206) (width 0.25) (layer "B.Cu") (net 19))
 (segment (start 162.1 71.4221) (end 162.1 74.3739) (width 0.25) (layer "B.Cu") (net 20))
 (segment (start 158.75 75.438) (end 161.036 75.438) (width 0.25) (layer "B.Cu") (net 20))
 (segment (start 162.1 74.3739) (end 161.036 75.438) (width 0.25) (layer "B.Cu") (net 20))
 (segment (start 158.75 70.358) (end 161.036 70.358) (width 0.25) (layer "B.Cu") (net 20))
 (segment (start 161.036 70.358) (end 162.1 71.4221) (width 0.25) (layer "B.Cu") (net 20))
 (segment (start 142.88 77.978) (end 145.796 77.978) (width 0.25) (layer "B.Cu") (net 10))
 (segment (start 145.33 71.8429) (end 144.533 72.6392) (width 0.25) (layer "F.Cu") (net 9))
 (segment (start 145.796 60.198) (end 147.324 61.7259) (width 0.25) (layer "F.Cu") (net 9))
 (segment (start 145.849 71.8429) (end 145.33 71.8429) (width 0.25) (layer "F.Cu") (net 9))
 (segment (start 144.533 72.6392) (end 144.533 73.7848) (width 0.25) (layer "F.Cu") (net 9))
 (segment (start 144.533 73.7848) (end 142.88 75.438) (width 0.25) (layer "F.Cu") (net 9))
 (segment (start 147.324 61.7259) (end 147.324 70.3677) (width 0.25) (layer "F.Cu") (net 9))
 (segment (start 147.324 70.3677) (end 145.849 71.8429) (width 0.25) (layer "F.Cu") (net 9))
 (segment (start 145.42 75.438) (end 145.796 75.438) (width 0.25) (layer "B.Cu") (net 8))
 (segment (start 142.88 72.898) (end 145.42 75.438) (width 0.25) (layer "B.Cu") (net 8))
 (segment (start 163.174 62.1378) (end 161.036 64.2754) (width 0.25) (layer "F.Cu") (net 7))
 (segment (start 161.036 64.2754) (end 161.036 65.278) (width 0.25) (layer "F.Cu") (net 7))
 (via (at 163.174 62.1378) (size 0.8) (drill 0.4) (layers "F.Cu" "B.Cu") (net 7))
 (segment (start 142.88 70.358) (end 141.555 69.0326) (width 0.25) (layer "B.Cu") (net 7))
 (segment (start 141.555 53.9146) (end 141.731 53.7385) (width 0.25) (layer "B.Cu") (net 7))
 (segment (start 141.555 69.0326) (end 141.555 53.9146) (width 0.25) (layer "B.Cu") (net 7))
 (segment (start 163.174 55.75) (end 163.174 62.1378) (width 0.25) (layer "B.Cu") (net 7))
 (segment (start 161.162 53.7385) (end 163.174 55.75) (width 0.25) (layer "B.Cu") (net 7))
 (segment (start 141.731 53.7385) (end 161.162 53.7385) (width 0.25) (layer "B.Cu") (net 7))
 (segment (start 142.88 67.818) (end 144.533 69.4712) (width 0.25) (layer "B.Cu") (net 6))
 (segment (start 144.533 69.4712) (end 144.533 71.6352) (width 0.25) (layer "B.Cu") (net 6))
 (segment (start 144.533 71.6352) (end 145.796 72.898) (width 0.25) (layer "B.Cu") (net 6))
 (segment (start 160.02 58.928) (end 161.32 58.928) (width 0.25) (layer "B.Cu") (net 26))
 (segment (start 158.75 57.658) (end 160.02 58.928) (width 0.25) (layer "B.Cu") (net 26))
 (segment (start 162.098 59.707) (end 162.098 66.7555) (width 0.25) (layer "B.Cu") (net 26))
 (segment (start 161.32 58.928) (end 162.098 59.707) (width 0.25) (layer "B.Cu") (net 26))
 (segment (start 162.098 66.7555) (end 161.036 67.818) (width 0.25) (layer "B.Cu") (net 26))
 (segment (start 162.132 59.1025) (end 161.036 60.198) (width 0.25) (layer "F.Cu") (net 27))
 (segment (start 160.02 56.388) (end 161.259 56.388) (width 0.25) (layer "F.Cu") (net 27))
 (segment (start 158.75 55.118) (end 160.02 56.388) (width 0.25) (layer "F.Cu") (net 27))
 (segment (start 162.132 57.2606) (end 162.132 59.1025) (width 0.25) (layer "F.Cu") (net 27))
 (segment (start 161.259 56.388) (end 162.132 57.2606) (width 0.25) (layer "F.Cu") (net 27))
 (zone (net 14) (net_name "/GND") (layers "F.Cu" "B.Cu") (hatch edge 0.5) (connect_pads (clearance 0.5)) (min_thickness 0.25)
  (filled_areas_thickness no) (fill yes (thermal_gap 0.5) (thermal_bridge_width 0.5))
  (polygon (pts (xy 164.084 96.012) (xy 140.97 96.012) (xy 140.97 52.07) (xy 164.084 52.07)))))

